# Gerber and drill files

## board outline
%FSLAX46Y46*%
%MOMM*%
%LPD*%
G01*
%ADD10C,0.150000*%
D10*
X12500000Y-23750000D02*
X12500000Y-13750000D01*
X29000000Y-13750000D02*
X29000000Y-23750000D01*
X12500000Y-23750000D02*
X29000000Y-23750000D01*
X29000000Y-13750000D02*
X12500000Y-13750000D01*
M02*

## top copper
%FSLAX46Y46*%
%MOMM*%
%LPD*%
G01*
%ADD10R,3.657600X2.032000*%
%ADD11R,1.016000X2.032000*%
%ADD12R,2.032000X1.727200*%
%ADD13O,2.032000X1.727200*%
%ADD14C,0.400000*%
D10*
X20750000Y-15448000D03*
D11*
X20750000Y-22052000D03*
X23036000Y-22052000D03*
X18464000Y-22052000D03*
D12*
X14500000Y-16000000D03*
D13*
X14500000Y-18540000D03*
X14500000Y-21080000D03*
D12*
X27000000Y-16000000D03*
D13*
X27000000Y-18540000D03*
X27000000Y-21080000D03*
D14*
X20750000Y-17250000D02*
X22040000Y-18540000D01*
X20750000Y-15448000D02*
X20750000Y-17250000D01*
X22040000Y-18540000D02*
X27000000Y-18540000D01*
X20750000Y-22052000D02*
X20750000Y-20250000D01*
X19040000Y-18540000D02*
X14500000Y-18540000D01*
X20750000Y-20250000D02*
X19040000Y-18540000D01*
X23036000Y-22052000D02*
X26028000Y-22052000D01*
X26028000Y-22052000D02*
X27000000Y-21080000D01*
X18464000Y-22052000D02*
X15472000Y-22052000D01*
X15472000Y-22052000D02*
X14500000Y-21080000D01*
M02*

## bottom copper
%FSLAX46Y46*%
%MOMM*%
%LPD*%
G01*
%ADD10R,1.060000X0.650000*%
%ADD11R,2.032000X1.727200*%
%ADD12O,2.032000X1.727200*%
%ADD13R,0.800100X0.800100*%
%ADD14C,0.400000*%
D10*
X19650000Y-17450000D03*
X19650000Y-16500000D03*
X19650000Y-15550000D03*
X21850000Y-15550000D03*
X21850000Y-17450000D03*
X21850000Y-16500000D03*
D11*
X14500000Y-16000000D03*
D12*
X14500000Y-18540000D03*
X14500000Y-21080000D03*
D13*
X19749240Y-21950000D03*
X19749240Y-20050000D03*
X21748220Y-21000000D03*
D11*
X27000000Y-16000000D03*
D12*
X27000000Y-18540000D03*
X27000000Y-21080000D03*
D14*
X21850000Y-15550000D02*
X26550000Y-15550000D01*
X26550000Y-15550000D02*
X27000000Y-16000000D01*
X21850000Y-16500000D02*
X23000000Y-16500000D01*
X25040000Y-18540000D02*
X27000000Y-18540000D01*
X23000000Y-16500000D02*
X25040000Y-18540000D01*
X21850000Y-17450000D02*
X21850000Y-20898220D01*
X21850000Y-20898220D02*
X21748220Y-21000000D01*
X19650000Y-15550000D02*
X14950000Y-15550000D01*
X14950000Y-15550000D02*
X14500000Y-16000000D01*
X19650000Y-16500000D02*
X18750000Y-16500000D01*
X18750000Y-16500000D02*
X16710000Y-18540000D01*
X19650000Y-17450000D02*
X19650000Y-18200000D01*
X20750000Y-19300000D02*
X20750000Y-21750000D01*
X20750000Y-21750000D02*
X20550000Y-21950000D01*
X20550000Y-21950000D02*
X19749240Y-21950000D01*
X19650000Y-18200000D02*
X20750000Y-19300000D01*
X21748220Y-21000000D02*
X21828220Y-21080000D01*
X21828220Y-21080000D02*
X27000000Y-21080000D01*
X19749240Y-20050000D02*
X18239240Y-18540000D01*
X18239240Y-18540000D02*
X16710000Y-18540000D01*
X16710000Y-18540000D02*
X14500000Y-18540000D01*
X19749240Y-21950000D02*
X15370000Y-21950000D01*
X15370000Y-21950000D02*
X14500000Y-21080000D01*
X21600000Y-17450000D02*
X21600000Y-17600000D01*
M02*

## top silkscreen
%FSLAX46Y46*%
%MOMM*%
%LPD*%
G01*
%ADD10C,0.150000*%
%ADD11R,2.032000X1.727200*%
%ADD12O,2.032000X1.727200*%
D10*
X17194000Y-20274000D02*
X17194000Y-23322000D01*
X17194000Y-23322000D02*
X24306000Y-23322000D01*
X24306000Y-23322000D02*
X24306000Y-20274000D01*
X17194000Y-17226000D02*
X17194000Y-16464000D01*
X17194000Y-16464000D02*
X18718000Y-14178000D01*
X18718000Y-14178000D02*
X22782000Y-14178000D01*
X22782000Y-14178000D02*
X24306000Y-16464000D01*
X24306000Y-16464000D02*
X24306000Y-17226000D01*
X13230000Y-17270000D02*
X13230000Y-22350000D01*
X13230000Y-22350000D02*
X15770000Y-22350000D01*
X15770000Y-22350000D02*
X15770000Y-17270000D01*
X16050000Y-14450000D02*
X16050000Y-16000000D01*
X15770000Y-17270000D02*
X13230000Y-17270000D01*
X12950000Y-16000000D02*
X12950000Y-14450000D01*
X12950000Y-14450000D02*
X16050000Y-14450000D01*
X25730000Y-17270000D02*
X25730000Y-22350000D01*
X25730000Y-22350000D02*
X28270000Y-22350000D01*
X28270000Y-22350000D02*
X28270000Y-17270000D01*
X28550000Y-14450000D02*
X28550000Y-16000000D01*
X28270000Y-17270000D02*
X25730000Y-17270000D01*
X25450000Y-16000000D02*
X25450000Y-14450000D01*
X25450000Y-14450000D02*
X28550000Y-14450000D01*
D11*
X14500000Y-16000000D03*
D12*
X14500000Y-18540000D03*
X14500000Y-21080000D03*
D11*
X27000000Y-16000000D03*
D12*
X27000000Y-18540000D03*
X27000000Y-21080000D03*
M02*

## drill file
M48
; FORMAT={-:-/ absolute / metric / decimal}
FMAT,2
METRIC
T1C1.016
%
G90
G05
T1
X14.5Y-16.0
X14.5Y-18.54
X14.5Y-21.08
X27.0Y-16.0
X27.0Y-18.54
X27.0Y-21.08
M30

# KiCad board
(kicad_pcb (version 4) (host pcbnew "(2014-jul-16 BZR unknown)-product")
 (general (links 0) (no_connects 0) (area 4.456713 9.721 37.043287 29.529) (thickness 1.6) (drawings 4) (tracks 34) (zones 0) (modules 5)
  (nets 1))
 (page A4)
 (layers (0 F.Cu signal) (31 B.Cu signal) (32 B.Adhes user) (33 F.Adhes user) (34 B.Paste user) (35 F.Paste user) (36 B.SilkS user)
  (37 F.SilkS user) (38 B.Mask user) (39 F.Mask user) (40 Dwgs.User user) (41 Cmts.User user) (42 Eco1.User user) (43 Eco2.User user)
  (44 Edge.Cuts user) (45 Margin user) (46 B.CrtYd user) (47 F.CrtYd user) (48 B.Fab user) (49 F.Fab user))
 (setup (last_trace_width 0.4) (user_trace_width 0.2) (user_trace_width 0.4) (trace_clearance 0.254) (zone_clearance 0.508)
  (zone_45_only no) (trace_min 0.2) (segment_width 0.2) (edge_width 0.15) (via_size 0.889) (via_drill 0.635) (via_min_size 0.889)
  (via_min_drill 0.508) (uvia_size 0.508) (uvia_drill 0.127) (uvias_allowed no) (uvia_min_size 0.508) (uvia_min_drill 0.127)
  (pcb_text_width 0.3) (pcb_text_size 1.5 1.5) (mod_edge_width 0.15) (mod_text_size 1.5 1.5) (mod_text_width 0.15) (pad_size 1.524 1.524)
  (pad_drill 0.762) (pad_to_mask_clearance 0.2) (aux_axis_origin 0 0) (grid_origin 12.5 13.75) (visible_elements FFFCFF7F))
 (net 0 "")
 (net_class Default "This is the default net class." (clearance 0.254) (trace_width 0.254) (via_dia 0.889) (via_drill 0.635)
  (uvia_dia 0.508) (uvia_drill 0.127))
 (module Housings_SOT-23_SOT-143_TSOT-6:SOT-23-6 (layer B.Cu) (at 20.75 16.5)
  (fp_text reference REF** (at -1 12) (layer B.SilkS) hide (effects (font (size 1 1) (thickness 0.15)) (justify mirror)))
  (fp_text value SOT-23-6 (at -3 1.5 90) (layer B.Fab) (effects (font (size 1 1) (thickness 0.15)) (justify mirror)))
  (pad 1 smd rect (at -1.1 0.95) (size 1.06 0.65) (layers B.Cu B.Paste B.Mask))
  (pad 2 smd rect (at -1.1 0) (size 1.06 0.65) (layers B.Cu B.Paste B.Mask))
  (pad 3 smd rect (at -1.1 -0.95) (size 1.06 0.65) (layers B.Cu B.Paste B.Mask))
  (pad 4 smd rect (at 1.1 -0.95) (size 1.06 0.65) (layers B.Cu B.Paste B.Mask))
  (pad 6 smd rect (at 1.1 0.95) (size 1.06 0.65) (layers B.Cu B.Paste B.Mask))
  (pad 5 smd rect (at 1.1 0) (size 1.06 0.65) (layers B.Cu B.Paste B.Mask)))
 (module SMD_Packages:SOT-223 (layer F.Cu) (at 20.75 18.75)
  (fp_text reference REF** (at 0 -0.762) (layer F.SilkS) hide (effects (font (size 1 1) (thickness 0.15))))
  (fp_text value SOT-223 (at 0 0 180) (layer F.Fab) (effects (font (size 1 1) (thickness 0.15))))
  (fp_line (start -3.556 1.524) (end -3.556 4.572) (layer F.SilkS) (width 0.15))
  (fp_line (start -3.556 4.572) (end 3.556 4.572) (layer F.SilkS) (width 0.15))
  (fp_line (start 3.556 4.572) (end 3.556 1.524) (layer F.SilkS) (width 0.15))
  (fp_line (start -3.556 -1.524) (end -3.556 -2.286) (layer F.SilkS) (width 0.15))
  (fp_line (start -3.556 -2.286) (end -2.032 -4.572) (layer F.SilkS) (width 0.15))
  (fp_line (start -2.032 -4.572) (end 2.032 -4.572) (layer F.SilkS) (width 0.15))
  (fp_line (start 2.032 -4.572) (end 3.556 -2.286) (layer F.SilkS) (width 0.15))
  (fp_line (start 3.556 -2.286) (end 3.556 -1.524) (layer F.SilkS) (width 0.15))
  (pad 4 smd rect (at 0 -3.302) (size 3.6576 2.032) (layers F.Cu F.Paste F.Mask))
  (pad 2 smd rect (at 0 3.302) (size 1.016 2.032) (layers F.Cu F.Paste F.Mask))
  (pad 3 smd rect (at 2.286 3.302) (size 1.016 2.032) (layers F.Cu F.Paste F.Mask))
  (pad 1 smd rect (at -2.286 3.302) (size 1.016 2.032) (layers F.Cu F.Paste F.Mask)))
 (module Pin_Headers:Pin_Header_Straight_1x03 (layer F.Cu) (at 14.5 16)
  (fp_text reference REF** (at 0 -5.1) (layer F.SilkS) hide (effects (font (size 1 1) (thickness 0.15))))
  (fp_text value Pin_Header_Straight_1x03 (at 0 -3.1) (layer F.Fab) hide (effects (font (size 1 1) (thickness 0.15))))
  (fp_line (start -1.27 1.27) (end -1.27 6.35) (layer F.SilkS) (width 0.15))
  (fp_line (start -1.27 6.35) (end 1.27 6.35) (layer F.SilkS) (width 0.15))
  (fp_line (start 1.27 6.35) (end 1.27 1.27) (layer F.SilkS) (width 0.15))
  (fp_line (start 1.55 -1.55) (end 1.55 0) (layer F.SilkS) (width 0.15))
  (fp_line (start 1.27 1.27) (end -1.27 1.27) (layer F.SilkS) (width 0.15))
  (fp_line (start -1.55 0) (end -1.55 -1.55) (layer F.SilkS) (width 0.15))
  (fp_line (start -1.55 -1.55) (end 1.55 -1.55) (layer F.SilkS) (width 0.15))
  (pad 1 thru_hole rect (at 0 0) (size 2.032 1.7272) (drill 1.016) (layers *.Cu *.Mask F.SilkS))
  (pad 2 thru_hole oval (at 0 2.54) (size 2.032 1.7272) (drill 1.016) (layers *.Cu *.Mask F.SilkS))
  (pad 3 thru_hole oval (at 0 5.08) (size 2.032 1.7272) (drill 1.016) (layers *.Cu *.Mask F.SilkS)))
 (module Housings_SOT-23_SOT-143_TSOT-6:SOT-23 (layer B.Cu) (at 20.75 21 90)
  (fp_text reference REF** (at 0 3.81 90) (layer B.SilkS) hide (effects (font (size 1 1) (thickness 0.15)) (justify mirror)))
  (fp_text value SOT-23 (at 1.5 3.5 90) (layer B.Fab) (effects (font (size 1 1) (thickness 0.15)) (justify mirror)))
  (pad 1 smd rect (at -0.95 -1.00076 90) (size 0.8001 0.8001) (layers B.Cu B.Paste B.Mask))
  (pad 2 smd rect (at 0.95 -1.00076 90) (size 0.8001 0.8001) (layers B.Cu B.Paste B.Mask))
  (pad 3 smd rect (at 0 0.99822 90) (size 0.8001 0.8001) (layers B.Cu B.Paste B.Mask)))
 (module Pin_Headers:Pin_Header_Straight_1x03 (layer F.Cu) (at 27 16)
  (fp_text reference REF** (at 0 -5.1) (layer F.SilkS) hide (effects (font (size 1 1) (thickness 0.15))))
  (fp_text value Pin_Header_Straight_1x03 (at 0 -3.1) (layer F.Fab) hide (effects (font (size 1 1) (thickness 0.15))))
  (fp_line (start -1.27 1.27) (end -1.27 6.35) (layer F.SilkS) (width 0.15))
  (fp_line (start -1.27 6.35) (end 1.27 6.35) (layer F.SilkS) (width 0.15))
  (fp_line (start 1.27 6.35) (end 1.27 1.27) (layer F.SilkS) (width 0.15))
  (fp_line (start 1.55 -1.55) (end 1.55 0) (layer F.SilkS) (width 0.15))
  (fp_line (start 1.27 1.27) (end -1.27 1.27) (layer F.SilkS) (width 0.15))
  (fp_line (start -1.55 0) (end -1.55 -1.55) (layer F.SilkS) (width 0.15))
  (fp_line (start -1.55 -1.55) (end 1.55 -1.55) (layer F.SilkS) (width 0.15))
  (pad 1 thru_hole rect (at 0 0) (size 2.032 1.7272) (drill 1.016) (layers *.Cu *.Mask F.SilkS))
  (pad 2 thru_hole oval (at 0 2.54) (size 2.032 1.7272) (drill 1.016) (layers *.Cu *.Mask F.SilkS))
  (pad 3 thru_hole oval (at 0 5.08) (size 2.032 1.7272) (drill 1.016) (layers *.Cu *.Mask F.SilkS)))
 (gr_line (start 12.5 23.75) (end 12.5 13.75) (angle 90) (layer Edge.Cuts) (width 0.15))
 (gr_line (start 29 13.75) (end 29 23.75) (angle 90) (layer Edge.Cuts) (width 0.15))
 (gr_line (start 12.5 23.75) (end 29 23.75) (angle 90) (layer Edge.Cuts) (width 0.15))
 (gr_line (start 29 13.75) (end 12.5 13.75) (angle 90) (layer Edge.Cuts) (width 0.15))
 (segment (start 21.85 15.55) (end 26.55 15.55) (width 0.4) (layer B.Cu) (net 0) (status C00000))
 (segment (start 26.55 15.55) (end 27 16) (width 0.4) (layer B.Cu) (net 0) (status C00000))
 (segment (start 21.85 16.5) (end 23 16.5) (width 0.4) (layer B.Cu) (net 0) (status 400000))
 (segment (start 25.04 18.54) (end 27 18.54) (width 0.4) (layer B.Cu) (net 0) (status 800000))
 (segment (start 23 16.5) (end 25.04 18.54) (width 0.4) (layer B.Cu) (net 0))
 (segment (start 21.85 17.45) (end 21.85 20.89822) (width 0.4) (layer B.Cu) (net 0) (status C00000))
 (segment (start 21.85 20.89822) (end 21.74822 21) (width 0.4) (layer B.Cu) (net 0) (status C00000))
 (segment (start 20.75 17.25) (end 22.04 18.54) (width 0.4) (layer F.Cu) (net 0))
 (segment (start 20.75 15.448) (end 20.75 17.25) (width 0.4) (layer F.Cu) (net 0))
 (segment (start 22.04 18.54) (end 27 18.54) (width 0.4) (layer F.Cu) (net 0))
 (segment (start 19.65 15.55) (end 14.95 15.55) (width 0.4) (layer B.Cu) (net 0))
 (segment (start 14.95 15.55) (end 14.5 16) (width 0.4) (layer B.Cu) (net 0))
 (segment (start 19.65 16.5) (end 18.75 16.5) (width 0.4) (layer B.Cu) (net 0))
 (segment (start 18.75 16.5) (end 16.71 18.54) (width 0.4) (layer B.Cu) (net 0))
 (segment (start 19.65 17.45) (end 19.65 18.2) (width 0.4) (layer B.Cu) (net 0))
 (segment (start 20.75 19.3) (end 20.75 21.75) (width 0.4) (layer B.Cu) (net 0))
 (segment (start 20.75 21.75) (end 20.55 21.95) (width 0.4) (layer B.Cu) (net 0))
 (segment (start 20.55 21.95) (end 19.74924 21.95) (width 0.4) (layer B.Cu) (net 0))
 (segment (start 19.65 18.2) (end 20.75 19.3) (width 0.4) (layer B.Cu) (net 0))
 (segment (start 21.74822 21) (end 21.82822 21.08) (width 0.4) (layer B.Cu) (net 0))
 (segment (start 21.82822 21.08) (end 27 21.08) (width 0.4) (layer B.Cu) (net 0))
 (segment (start 19.74924 20.05) (end 18.23924 18.54) (width 0.4) (layer B.Cu) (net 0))
 (segment (start 18.23924 18.54) (end 16.71 18.54) (width 0.4) (layer B.Cu) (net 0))
 (segment (start 16.71 18.54) (end 14.5 18.54) (width 0.4) (layer B.Cu) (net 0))
 (segment (start 19.74924 21.95) (end 15.37 21.95) (width 0.4) (layer B.Cu) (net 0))
 (segment (start 15.37 21.95) (end 14.5 21.08) (width 0.4) (layer B.Cu) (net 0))
 (segment (start 20.75 22.052) (end 20.75 20.25) (width 0.4) (layer F.Cu) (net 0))
 (segment (start 19.04 18.54) (end 14.5 18.54) (width 0.4) (layer F.Cu) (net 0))
 (segment (start 20.75 20.25) (end 19.04 18.54) (width 0.4) (layer F.Cu) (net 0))
 (segment (start 23.036 22.052) (end 26.028 22.052) (width 0.4) (layer F.Cu) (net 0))
 (segment (start 26.028 22.052) (end 27 21.08) (width 0.4) (layer F.Cu) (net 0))
 (segment (start 18.464 22.052) (end 15.472 22.052) (width 0.4) (layer F.Cu) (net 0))
 (segment (start 15.472 22.052) (end 14.5 21.08) (width 0.4) (layer F.Cu) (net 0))
 (segment (start 21.6 17.45) (end 21.6 17.6) (width 0.4) (layer B.Cu) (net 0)))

